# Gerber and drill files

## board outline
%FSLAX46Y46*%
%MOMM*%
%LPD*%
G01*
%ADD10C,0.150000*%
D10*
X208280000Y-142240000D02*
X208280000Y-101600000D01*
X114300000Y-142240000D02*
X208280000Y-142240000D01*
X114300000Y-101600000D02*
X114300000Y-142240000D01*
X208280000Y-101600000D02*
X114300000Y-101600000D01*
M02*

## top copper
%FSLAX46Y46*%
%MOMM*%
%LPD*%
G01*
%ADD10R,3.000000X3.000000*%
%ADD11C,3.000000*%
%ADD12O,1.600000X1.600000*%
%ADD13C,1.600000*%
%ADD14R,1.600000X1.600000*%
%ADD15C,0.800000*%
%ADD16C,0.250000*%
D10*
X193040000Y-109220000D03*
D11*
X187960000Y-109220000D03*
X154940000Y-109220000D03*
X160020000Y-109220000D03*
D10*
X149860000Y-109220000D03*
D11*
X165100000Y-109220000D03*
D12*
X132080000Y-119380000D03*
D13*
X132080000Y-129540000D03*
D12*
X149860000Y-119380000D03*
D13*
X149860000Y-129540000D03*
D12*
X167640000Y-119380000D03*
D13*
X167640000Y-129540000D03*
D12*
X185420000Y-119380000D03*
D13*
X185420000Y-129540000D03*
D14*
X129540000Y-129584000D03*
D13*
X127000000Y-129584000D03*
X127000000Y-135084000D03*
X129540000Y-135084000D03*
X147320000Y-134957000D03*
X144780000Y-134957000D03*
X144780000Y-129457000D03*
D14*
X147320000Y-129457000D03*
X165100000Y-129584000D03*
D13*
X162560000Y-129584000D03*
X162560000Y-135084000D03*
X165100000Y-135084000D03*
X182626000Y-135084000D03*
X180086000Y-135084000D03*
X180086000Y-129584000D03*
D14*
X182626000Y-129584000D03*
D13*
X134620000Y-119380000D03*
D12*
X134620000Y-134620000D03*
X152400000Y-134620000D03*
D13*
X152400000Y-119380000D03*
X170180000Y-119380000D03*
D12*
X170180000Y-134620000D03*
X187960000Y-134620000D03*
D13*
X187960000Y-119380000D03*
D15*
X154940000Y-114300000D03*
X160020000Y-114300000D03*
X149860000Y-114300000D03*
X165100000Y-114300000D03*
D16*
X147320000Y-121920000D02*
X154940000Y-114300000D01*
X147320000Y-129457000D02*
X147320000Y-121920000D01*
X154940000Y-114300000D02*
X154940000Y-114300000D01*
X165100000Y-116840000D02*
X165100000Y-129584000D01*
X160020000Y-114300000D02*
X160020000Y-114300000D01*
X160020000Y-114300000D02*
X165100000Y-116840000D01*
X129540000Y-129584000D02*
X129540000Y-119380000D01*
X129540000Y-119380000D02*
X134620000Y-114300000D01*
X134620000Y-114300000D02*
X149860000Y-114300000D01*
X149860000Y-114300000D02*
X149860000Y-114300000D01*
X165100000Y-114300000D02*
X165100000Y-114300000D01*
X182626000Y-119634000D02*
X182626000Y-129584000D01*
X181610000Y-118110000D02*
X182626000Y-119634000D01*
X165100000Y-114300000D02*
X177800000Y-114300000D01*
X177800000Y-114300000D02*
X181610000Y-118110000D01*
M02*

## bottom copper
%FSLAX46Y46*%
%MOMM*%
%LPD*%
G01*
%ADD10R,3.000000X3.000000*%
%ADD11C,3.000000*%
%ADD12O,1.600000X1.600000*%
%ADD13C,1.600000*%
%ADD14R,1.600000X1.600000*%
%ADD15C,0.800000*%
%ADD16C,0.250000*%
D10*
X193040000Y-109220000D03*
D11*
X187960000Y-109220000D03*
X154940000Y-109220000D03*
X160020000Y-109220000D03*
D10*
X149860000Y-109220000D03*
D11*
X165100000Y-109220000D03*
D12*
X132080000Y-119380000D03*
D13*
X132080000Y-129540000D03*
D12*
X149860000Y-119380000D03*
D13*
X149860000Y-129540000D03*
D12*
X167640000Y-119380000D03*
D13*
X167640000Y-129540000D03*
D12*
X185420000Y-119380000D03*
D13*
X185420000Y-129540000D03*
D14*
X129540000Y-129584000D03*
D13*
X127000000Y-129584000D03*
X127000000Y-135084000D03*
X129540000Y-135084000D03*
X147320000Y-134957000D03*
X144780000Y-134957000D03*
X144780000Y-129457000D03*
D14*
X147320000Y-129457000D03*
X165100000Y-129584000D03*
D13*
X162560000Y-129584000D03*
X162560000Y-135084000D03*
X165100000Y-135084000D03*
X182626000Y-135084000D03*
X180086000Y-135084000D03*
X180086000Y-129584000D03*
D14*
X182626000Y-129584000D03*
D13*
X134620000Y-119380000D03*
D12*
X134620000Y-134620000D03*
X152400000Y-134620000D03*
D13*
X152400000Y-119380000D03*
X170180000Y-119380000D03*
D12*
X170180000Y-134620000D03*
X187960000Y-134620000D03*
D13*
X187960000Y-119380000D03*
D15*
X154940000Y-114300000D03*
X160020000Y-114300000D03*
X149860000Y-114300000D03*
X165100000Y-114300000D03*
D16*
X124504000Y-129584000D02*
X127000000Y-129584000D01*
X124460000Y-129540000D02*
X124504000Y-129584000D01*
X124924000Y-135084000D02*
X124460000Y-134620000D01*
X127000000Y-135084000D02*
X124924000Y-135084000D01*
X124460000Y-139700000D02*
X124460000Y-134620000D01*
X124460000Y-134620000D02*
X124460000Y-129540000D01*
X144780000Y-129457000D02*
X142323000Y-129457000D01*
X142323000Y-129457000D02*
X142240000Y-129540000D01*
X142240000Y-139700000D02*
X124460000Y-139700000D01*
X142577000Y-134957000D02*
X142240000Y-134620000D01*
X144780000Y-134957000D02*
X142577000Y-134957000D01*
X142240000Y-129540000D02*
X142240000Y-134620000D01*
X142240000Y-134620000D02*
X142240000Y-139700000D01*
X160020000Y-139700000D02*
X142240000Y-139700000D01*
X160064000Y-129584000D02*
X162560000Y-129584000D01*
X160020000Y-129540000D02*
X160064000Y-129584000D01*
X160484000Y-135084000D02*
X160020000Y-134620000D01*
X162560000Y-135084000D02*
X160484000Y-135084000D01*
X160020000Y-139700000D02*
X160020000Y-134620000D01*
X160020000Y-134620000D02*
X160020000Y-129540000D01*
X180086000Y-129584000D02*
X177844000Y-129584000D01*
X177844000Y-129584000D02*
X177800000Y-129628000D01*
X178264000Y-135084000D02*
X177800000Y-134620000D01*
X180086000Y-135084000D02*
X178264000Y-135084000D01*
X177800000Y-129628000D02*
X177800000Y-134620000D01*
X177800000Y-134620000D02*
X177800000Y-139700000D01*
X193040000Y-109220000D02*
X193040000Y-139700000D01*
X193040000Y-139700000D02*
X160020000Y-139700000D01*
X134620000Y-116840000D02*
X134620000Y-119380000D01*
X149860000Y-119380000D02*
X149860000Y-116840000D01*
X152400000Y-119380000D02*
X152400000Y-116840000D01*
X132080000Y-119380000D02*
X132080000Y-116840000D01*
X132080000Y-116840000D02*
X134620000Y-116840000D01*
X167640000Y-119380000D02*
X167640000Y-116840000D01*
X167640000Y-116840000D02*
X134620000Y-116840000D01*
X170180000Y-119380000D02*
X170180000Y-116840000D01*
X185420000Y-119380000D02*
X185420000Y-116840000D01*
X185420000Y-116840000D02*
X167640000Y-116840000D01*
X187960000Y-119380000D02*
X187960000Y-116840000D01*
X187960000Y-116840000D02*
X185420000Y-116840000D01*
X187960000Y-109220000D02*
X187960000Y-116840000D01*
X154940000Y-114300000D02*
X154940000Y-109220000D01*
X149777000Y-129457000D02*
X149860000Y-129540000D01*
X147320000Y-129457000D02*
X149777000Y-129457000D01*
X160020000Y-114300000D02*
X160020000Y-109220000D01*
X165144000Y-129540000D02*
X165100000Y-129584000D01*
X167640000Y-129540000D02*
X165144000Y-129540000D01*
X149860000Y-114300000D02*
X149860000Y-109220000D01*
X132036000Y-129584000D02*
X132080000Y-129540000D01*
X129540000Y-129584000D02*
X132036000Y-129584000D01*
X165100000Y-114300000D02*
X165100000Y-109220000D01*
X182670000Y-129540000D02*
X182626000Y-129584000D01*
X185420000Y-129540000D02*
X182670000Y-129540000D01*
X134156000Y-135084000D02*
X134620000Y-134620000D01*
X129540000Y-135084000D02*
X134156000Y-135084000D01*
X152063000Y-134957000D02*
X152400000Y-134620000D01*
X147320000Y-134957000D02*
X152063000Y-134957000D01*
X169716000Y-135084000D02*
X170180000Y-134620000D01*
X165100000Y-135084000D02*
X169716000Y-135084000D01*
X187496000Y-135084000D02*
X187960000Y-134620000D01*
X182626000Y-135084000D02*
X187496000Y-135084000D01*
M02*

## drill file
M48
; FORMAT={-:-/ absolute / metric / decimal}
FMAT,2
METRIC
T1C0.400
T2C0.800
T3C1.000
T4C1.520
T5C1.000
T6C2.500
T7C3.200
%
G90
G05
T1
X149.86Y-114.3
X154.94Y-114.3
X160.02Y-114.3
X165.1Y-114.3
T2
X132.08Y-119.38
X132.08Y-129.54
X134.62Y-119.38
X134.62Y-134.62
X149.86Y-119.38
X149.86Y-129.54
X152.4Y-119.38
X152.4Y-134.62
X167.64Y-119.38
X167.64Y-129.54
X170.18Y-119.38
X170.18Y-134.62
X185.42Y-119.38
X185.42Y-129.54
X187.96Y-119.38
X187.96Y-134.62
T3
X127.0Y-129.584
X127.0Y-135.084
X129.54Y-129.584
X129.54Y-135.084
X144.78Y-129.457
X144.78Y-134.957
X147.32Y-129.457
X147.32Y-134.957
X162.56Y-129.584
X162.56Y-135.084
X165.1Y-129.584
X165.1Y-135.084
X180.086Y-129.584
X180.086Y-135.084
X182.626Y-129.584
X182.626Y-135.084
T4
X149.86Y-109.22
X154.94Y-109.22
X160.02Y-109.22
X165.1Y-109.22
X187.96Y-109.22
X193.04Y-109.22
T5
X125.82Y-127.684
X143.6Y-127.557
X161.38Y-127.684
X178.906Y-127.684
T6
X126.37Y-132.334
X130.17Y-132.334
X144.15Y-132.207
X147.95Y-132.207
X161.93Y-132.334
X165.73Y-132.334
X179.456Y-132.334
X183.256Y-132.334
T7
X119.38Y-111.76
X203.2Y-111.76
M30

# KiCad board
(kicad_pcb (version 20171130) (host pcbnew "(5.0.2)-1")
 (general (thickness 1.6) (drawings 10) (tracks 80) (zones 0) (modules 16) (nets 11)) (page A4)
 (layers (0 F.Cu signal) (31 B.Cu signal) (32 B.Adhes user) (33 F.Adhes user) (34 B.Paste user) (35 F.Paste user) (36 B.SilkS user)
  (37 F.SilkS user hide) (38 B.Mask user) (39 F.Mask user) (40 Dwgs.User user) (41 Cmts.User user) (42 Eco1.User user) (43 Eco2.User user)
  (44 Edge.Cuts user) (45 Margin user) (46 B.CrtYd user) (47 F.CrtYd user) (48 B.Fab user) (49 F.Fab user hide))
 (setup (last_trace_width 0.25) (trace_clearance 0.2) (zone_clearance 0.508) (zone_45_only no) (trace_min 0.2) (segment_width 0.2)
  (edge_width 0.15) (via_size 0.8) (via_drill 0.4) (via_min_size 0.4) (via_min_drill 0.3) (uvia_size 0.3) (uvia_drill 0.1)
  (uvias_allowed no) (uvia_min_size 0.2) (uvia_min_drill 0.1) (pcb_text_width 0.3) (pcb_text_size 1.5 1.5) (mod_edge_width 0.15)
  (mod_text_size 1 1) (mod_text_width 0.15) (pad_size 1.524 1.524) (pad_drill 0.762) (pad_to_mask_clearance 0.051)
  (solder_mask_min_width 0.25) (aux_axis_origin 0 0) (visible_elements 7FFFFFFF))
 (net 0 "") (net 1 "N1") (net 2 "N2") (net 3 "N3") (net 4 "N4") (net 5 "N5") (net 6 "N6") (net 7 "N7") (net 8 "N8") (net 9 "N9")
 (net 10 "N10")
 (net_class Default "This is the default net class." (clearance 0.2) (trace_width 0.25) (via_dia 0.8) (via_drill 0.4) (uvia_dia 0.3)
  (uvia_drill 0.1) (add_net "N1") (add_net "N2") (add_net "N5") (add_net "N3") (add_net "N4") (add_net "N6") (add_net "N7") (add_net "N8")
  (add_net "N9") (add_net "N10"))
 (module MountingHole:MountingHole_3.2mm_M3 (layer F.Cu) (at 203.2 111.76)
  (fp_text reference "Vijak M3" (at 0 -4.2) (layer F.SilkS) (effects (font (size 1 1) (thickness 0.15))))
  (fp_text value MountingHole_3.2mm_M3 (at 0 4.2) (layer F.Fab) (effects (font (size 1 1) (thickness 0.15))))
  (pad 1 np_thru_hole circle (at 0 0) (size 3.2 3.2) (drill 3.2) (layers *.Cu *.Mask)))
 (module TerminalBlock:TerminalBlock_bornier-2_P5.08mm (layer F.Cu) (at 193.04 109.22 180)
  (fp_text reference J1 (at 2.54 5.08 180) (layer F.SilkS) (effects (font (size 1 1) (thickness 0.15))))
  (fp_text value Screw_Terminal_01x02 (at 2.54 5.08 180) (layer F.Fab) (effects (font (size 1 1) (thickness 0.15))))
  (pad 1 thru_hole rect (at 0 0 180) (size 3 3) (drill 1.52) (layers *.Cu *.Mask) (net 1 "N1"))
  (pad 2 thru_hole circle (at 5.08 0 180) (size 3 3) (drill 1.52) (layers *.Cu *.Mask) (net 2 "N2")))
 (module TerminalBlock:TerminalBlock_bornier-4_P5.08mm (layer F.Cu) (at 149.86 109.22)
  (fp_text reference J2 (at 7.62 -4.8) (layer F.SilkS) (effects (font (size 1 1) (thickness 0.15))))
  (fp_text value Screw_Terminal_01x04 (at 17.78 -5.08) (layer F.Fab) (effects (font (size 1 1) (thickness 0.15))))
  (pad 2 thru_hole circle (at 5.08 0) (size 3 3) (drill 1.52) (layers *.Cu *.Mask) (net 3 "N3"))
  (pad 3 thru_hole circle (at 10.16 0) (size 3 3) (drill 1.52) (layers *.Cu *.Mask) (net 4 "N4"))
  (pad 1 thru_hole rect (at 0 0) (size 3 3) (drill 1.52) (layers *.Cu *.Mask) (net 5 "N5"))
  (pad 4 thru_hole circle (at 15.24 0) (size 3 3) (drill 1.52) (layers *.Cu *.Mask) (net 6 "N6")))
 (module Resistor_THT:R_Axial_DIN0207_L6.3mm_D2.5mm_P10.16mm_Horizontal (layer F.Cu) (at 132.08 129.54 90)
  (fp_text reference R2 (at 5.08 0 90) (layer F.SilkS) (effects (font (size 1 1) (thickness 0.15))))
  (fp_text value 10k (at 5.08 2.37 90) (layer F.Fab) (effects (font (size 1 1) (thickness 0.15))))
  (pad 2 thru_hole oval (at 10.16 0 90) (size 1.6 1.6) (drill 0.8) (layers *.Cu *.Mask) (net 2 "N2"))
  (pad 1 thru_hole circle (at 0 0 90) (size 1.6 1.6) (drill 0.8) (layers *.Cu *.Mask) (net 5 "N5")))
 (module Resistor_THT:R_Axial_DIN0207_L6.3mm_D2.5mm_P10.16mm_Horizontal (layer F.Cu) (at 149.86 129.54 90)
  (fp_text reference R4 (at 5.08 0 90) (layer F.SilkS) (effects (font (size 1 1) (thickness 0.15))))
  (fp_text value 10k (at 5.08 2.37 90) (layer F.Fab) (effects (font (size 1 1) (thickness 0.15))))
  (pad 2 thru_hole oval (at 10.16 0 90) (size 1.6 1.6) (drill 0.8) (layers *.Cu *.Mask) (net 2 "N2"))
  (pad 1 thru_hole circle (at 0 0 90) (size 1.6 1.6) (drill 0.8) (layers *.Cu *.Mask) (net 3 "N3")))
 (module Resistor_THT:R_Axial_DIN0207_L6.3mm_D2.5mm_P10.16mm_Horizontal (layer F.Cu) (at 167.64 129.54 90)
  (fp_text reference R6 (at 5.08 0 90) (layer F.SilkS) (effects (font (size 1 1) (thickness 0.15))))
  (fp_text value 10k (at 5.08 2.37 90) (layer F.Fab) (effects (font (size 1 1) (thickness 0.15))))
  (pad 2 thru_hole oval (at 10.16 0 90) (size 1.6 1.6) (drill 0.8) (layers *.Cu *.Mask) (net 2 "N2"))
  (pad 1 thru_hole circle (at 0 0 90) (size 1.6 1.6) (drill 0.8) (layers *.Cu *.Mask) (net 4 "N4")))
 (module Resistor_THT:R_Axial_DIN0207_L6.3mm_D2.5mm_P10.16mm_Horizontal (layer F.Cu) (at 185.42 129.54 90)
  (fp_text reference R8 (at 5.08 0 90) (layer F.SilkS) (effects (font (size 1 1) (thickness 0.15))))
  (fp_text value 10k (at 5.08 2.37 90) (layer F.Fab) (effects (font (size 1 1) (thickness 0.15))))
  (pad 2 thru_hole oval (at 10.16 0 90) (size 1.6 1.6) (drill 0.8) (layers *.Cu *.Mask) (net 2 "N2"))
  (pad 1 thru_hole circle (at 0 0 90) (size 1.6 1.6) (drill 0.8) (layers *.Cu *.Mask) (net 6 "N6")))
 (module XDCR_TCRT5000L (layer F.Cu) (at 128.27 132.334 270)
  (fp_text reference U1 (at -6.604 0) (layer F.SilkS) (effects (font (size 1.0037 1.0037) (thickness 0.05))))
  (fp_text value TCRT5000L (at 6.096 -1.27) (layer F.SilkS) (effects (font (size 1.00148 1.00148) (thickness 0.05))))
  (pad 1 thru_hole rect (at -2.75 -1.27 270) (size 1.6 1.6) (drill 1) (layers *.Cu *.Mask) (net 5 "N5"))
  (pad 2 thru_hole circle (at -2.75 1.27 270) (size 1.6 1.6) (drill 1) (layers *.Cu *.Mask) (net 1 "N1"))
  (pad 3 thru_hole circle (at 2.75 1.27 270) (size 1.6 1.6) (drill 1) (layers *.Cu *.Mask) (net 1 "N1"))
  (pad 4 thru_hole circle (at 2.75 -1.27 270) (size 1.6 1.6) (drill 1) (layers *.Cu *.Mask) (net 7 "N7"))
  (pad Hole np_thru_hole circle (at 0 -1.9 270) (size 2.5 2.5) (drill 2.5) (layers *.Cu *.Mask F.SilkS))
  (pad Hole np_thru_hole circle (at 0 1.9 270) (size 2.5 2.5) (drill 2.5) (layers *.Cu *.Mask F.SilkS))
  (pad Hole np_thru_hole circle (at -4.65 2.45 270) (size 1 1) (drill 1) (layers *.Cu *.Mask F.SilkS)))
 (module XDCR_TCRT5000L (layer F.Cu) (at 146.05 132.207 270)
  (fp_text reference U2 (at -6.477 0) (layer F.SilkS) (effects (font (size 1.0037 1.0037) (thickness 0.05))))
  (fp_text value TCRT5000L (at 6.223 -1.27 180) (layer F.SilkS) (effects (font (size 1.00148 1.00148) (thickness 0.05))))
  (pad Hole np_thru_hole circle (at -4.65 2.45 270) (size 1 1) (drill 1) (layers *.Cu *.Mask F.SilkS))
  (pad Hole np_thru_hole circle (at 0 1.9 270) (size 2.5 2.5) (drill 2.5) (layers *.Cu *.Mask F.SilkS))
  (pad Hole np_thru_hole circle (at 0 -1.9 270) (size 2.5 2.5) (drill 2.5) (layers *.Cu *.Mask F.SilkS))
  (pad 4 thru_hole circle (at 2.75 -1.27 270) (size 1.6 1.6) (drill 1) (layers *.Cu *.Mask) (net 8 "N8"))
  (pad 3 thru_hole circle (at 2.75 1.27 270) (size 1.6 1.6) (drill 1) (layers *.Cu *.Mask) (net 1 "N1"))
  (pad 2 thru_hole circle (at -2.75 1.27 270) (size 1.6 1.6) (drill 1) (layers *.Cu *.Mask) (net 1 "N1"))
  (pad 1 thru_hole rect (at -2.75 -1.27 270) (size 1.6 1.6) (drill 1) (layers *.Cu *.Mask) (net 3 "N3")))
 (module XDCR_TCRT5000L (layer F.Cu) (at 163.83 132.334 270)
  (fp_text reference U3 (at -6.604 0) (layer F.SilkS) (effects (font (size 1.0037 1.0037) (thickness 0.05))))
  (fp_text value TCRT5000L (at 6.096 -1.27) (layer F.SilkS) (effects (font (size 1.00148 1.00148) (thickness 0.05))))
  (pad 1 thru_hole rect (at -2.75 -1.27 270) (size 1.6 1.6) (drill 1) (layers *.Cu *.Mask) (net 4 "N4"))
  (pad 2 thru_hole circle (at -2.75 1.27 270) (size 1.6 1.6) (drill 1) (layers *.Cu *.Mask) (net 1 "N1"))
  (pad 3 thru_hole circle (at 2.75 1.27 270) (size 1.6 1.6) (drill 1) (layers *.Cu *.Mask) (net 1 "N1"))
  (pad 4 thru_hole circle (at 2.75 -1.27 270) (size 1.6 1.6) (drill 1) (layers *.Cu *.Mask) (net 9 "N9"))
  (pad Hole np_thru_hole circle (at 0 -1.9 270) (size 2.5 2.5) (drill 2.5) (layers *.Cu *.Mask F.SilkS))
  (pad Hole np_thru_hole circle (at 0 1.9 270) (size 2.5 2.5) (drill 2.5) (layers *.Cu *.Mask F.SilkS))
  (pad Hole np_thru_hole circle (at -4.65 2.45 270) (size 1 1) (drill 1) (layers *.Cu *.Mask F.SilkS)))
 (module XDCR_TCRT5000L (layer F.Cu) (at 181.356 132.334 270)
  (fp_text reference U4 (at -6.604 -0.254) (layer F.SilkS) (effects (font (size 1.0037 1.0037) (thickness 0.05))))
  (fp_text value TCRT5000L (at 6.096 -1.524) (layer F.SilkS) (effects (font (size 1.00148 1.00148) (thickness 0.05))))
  (pad Hole np_thru_hole circle (at -4.65 2.45 270) (size 1 1) (drill 1) (layers *.Cu *.Mask F.SilkS))
  (pad Hole np_thru_hole circle (at 0 1.9 270) (size 2.5 2.5) (drill 2.5) (layers *.Cu *.Mask F.SilkS))
  (pad Hole np_thru_hole circle (at 0 -1.9 270) (size 2.5 2.5) (drill 2.5) (layers *.Cu *.Mask F.SilkS))
  (pad 4 thru_hole circle (at 2.75 -1.27 270) (size 1.6 1.6) (drill 1) (layers *.Cu *.Mask) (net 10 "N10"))
  (pad 3 thru_hole circle (at 2.75 1.27 270) (size 1.6 1.6) (drill 1) (layers *.Cu *.Mask) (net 1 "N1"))
  (pad 2 thru_hole circle (at -2.75 1.27 270) (size 1.6 1.6) (drill 1) (layers *.Cu *.Mask) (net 1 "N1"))
  (pad 1 thru_hole rect (at -2.75 -1.27 270) (size 1.6 1.6) (drill 1) (layers *.Cu *.Mask) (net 6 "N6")))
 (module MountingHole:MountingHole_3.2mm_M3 (layer F.Cu) (at 119.38 111.76)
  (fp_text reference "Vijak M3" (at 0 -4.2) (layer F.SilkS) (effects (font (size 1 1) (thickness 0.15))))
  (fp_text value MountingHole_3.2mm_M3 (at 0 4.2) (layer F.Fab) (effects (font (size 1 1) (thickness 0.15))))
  (pad 1 np_thru_hole circle (at 0 0) (size 3.2 3.2) (drill 3.2) (layers *.Cu *.Mask)))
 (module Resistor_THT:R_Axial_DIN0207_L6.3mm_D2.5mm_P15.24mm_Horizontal (layer F.Cu) (at 134.62 119.38 270)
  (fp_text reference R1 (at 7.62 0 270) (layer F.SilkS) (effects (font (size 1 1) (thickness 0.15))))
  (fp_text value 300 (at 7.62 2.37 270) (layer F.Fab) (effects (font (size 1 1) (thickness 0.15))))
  (pad 1 thru_hole circle (at 0 0 270) (size 1.6 1.6) (drill 0.8) (layers *.Cu *.Mask) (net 2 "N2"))
  (pad 2 thru_hole oval (at 15.24 0 270) (size 1.6 1.6) (drill 0.8) (layers *.Cu *.Mask) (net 7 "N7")))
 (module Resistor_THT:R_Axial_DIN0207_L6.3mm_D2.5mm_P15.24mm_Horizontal (layer F.Cu) (at 152.4 119.38 270)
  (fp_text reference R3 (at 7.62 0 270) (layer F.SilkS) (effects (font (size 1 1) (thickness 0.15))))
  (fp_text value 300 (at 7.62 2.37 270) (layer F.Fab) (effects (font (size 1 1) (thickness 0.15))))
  (pad 2 thru_hole oval (at 15.24 0 270) (size 1.6 1.6) (drill 0.8) (layers *.Cu *.Mask) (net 8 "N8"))
  (pad 1 thru_hole circle (at 0 0 270) (size 1.6 1.6) (drill 0.8) (layers *.Cu *.Mask) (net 2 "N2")))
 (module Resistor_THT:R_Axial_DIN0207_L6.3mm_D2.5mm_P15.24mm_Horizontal (layer F.Cu) (at 170.18 119.38 270)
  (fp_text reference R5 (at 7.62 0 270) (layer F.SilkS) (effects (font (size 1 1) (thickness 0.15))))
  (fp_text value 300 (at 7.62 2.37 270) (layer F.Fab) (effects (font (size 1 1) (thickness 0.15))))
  (pad 1 thru_hole circle (at 0 0 270) (size 1.6 1.6) (drill 0.8) (layers *.Cu *.Mask) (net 2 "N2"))
  (pad 2 thru_hole oval (at 15.24 0 270) (size 1.6 1.6) (drill 0.8) (layers *.Cu *.Mask) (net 9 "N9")))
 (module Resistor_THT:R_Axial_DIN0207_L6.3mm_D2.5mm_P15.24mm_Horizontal (layer F.Cu) (at 187.96 119.38 270)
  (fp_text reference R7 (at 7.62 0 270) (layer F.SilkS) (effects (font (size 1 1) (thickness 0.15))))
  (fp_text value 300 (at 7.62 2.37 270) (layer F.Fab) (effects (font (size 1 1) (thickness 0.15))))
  (pad 2 thru_hole oval (at 15.24 0 270) (size 1.6 1.6) (drill 0.8) (layers *.Cu *.Mask) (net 10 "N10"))
  (pad 1 thru_hole circle (at 0 0 270) (size 1.6 1.6) (drill 0.8) (layers *.Cu *.Mask) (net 2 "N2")))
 (gr_line (start 208.28 142.24) (end 208.28 101.6) (layer Edge.Cuts) (width 0.15))
 (gr_line (start 114.3 142.24) (end 208.28 142.24) (layer Edge.Cuts) (width 0.15))
 (gr_line (start 114.3 101.6) (end 114.3 142.24) (layer Edge.Cuts) (width 0.15))
 (gr_line (start 208.28 101.6) (end 114.3 101.6) (layer Edge.Cuts) (width 0.15))
 (segment (start 124.504 129.584) (end 127 129.584) (width 0.25) (layer B.Cu) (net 1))
 (segment (start 124.46 129.54) (end 124.504 129.584) (width 0.25) (layer B.Cu) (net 1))
 (segment (start 124.924 135.084) (end 124.46 134.62) (width 0.25) (layer B.Cu) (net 1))
 (segment (start 127 135.084) (end 124.924 135.084) (width 0.25) (layer B.Cu) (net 1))
 (segment (start 124.46 139.7) (end 124.46 134.62) (width 0.25) (layer B.Cu) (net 1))
 (segment (start 124.46 134.62) (end 124.46 129.54) (width 0.25) (layer B.Cu) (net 1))
 (segment (start 144.78 129.457) (end 142.323 129.457) (width 0.25) (layer B.Cu) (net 1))
 (segment (start 142.323 129.457) (end 142.24 129.54) (width 0.25) (layer B.Cu) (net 1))
 (segment (start 142.24 139.7) (end 124.46 139.7) (width 0.25) (layer B.Cu) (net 1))
 (segment (start 142.577 134.957) (end 142.24 134.62) (width 0.25) (layer B.Cu) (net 1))
 (segment (start 144.78 134.957) (end 142.577 134.957) (width 0.25) (layer B.Cu) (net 1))
 (segment (start 142.24 129.54) (end 142.24 134.62) (width 0.25) (layer B.Cu) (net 1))
 (segment (start 142.24 134.62) (end 142.24 139.7) (width 0.25) (layer B.Cu) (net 1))
 (segment (start 160.02 139.7) (end 142.24 139.7) (width 0.25) (layer B.Cu) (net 1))
 (segment (start 160.064 129.584) (end 162.56 129.584) (width 0.25) (layer B.Cu) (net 1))
 (segment (start 160.02 129.54) (end 160.064 129.584) (width 0.25) (layer B.Cu) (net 1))
 (segment (start 160.484 135.084) (end 160.02 134.62) (width 0.25) (layer B.Cu) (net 1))
 (segment (start 162.56 135.084) (end 160.484 135.084) (width 0.25) (layer B.Cu) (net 1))
 (segment (start 160.02 139.7) (end 160.02 134.62) (width 0.25) (layer B.Cu) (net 1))
 (segment (start 160.02 134.62) (end 160.02 129.54) (width 0.25) (layer B.Cu) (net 1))
 (segment (start 180.086 129.584) (end 177.844 129.584) (width 0.25) (layer B.Cu) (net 1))
 (segment (start 177.844 129.584) (end 177.8 129.628) (width 0.25) (layer B.Cu) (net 1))
 (segment (start 178.264 135.084) (end 177.8 134.62) (width 0.25) (layer B.Cu) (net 1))
 (segment (start 180.086 135.084) (end 178.264 135.084) (width 0.25) (layer B.Cu) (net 1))
 (segment (start 177.8 129.628) (end 177.8 134.62) (width 0.25) (layer B.Cu) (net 1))
 (segment (start 177.8 134.62) (end 177.8 139.7) (width 0.25) (layer B.Cu) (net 1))
 (segment (start 193.04 109.22) (end 193.04 139.7) (width 0.25) (layer B.Cu) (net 1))
 (segment (start 193.04 139.7) (end 160.02 139.7) (width 0.25) (layer B.Cu) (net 1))
 (segment (start 134.62 116.84) (end 134.62 119.38) (width 0.25) (layer B.Cu) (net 2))
 (segment (start 149.86 119.38) (end 149.86 116.84) (width 0.25) (layer B.Cu) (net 2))
 (segment (start 152.4 119.38) (end 152.4 116.84) (width 0.25) (layer B.Cu) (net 2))
 (segment (start 132.08 119.38) (end 132.08 116.84) (width 0.25) (layer B.Cu) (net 2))
 (segment (start 132.08 116.84) (end 134.62 116.84) (width 0.25) (layer B.Cu) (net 2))
 (segment (start 167.64 119.38) (end 167.64 116.84) (width 0.25) (layer B.Cu) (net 2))
 (segment (start 167.64 116.84) (end 134.62 116.84) (width 0.25) (layer B.Cu) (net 2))
 (segment (start 170.18 119.38) (end 170.18 116.84) (width 0.25) (layer B.Cu) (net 2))
 (segment (start 185.42 119.38) (end 185.42 116.84) (width 0.25) (layer B.Cu) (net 2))
 (segment (start 185.42 116.84) (end 167.64 116.84) (width 0.25) (layer B.Cu) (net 2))
 (segment (start 187.96 119.38) (end 187.96 116.84) (width 0.25) (layer B.Cu) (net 2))
 (segment (start 187.96 116.84) (end 185.42 116.84) (width 0.25) (layer B.Cu) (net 2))
 (segment (start 187.96 109.22) (end 187.96 116.84) (width 0.25) (layer B.Cu) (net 2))
 (segment (start 147.32 121.92) (end 154.94 114.3) (width 0.25) (layer F.Cu) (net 3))
 (segment (start 147.32 129.457) (end 147.32 121.92) (width 0.25) (layer F.Cu) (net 3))
 (segment (start 154.94 114.3) (end 154.94 114.3) (width 0.25) (layer F.Cu) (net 3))
 (via (at 154.94 114.3) (size 0.8) (drill 0.4) (layers F.Cu B.Cu) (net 3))
 (segment (start 154.94 114.3) (end 154.94 109.22) (width 0.25) (layer B.Cu) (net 3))
 (segment (start 149.777 129.457) (end 149.86 129.54) (width 0.25) (layer B.Cu) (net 3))
 (segment (start 147.32 129.457) (end 149.777 129.457) (width 0.25) (layer B.Cu) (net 3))
 (segment (start 165.1 116.84) (end 165.1 129.584) (width 0.25) (layer F.Cu) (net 4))
 (segment (start 160.02 114.3) (end 160.02 114.3) (width 0.25) (layer F.Cu) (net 4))
 (segment (start 160.02 114.3) (end 165.1 116.84) (width 0.25) (layer F.Cu) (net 4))
 (via (at 160.02 114.3) (size 0.8) (drill 0.4) (layers F.Cu B.Cu) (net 4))
 (segment (start 160.02 114.3) (end 160.02 109.22) (width 0.25) (layer B.Cu) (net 4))
 (segment (start 165.144 129.54) (end 165.1 129.584) (width 0.25) (layer B.Cu) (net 4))
 (segment (start 167.64 129.54) (end 165.144 129.54) (width 0.25) (layer B.Cu) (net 4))
 (segment (start 129.54 129.584) (end 129.54 119.38) (width 0.25) (layer F.Cu) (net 5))
 (segment (start 129.54 119.38) (end 134.62 114.3) (width 0.25) (layer F.Cu) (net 5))
 (segment (start 134.62 114.3) (end 149.86 114.3) (width 0.25) (layer F.Cu) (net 5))
 (segment (start 149.86 114.3) (end 149.86 114.3) (width 0.25) (layer F.Cu) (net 5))
 (via (at 149.86 114.3) (size 0.8) (drill 0.4) (layers F.Cu B.Cu) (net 5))
 (segment (start 149.86 114.3) (end 149.86 109.22) (width 0.25) (layer B.Cu) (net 5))
 (segment (start 132.036 129.584) (end 132.08 129.54) (width 0.25) (layer B.Cu) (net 5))
 (segment (start 129.54 129.584) (end 132.036 129.584) (width 0.25) (layer B.Cu) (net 5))
 (segment (start 165.1 114.3) (end 165.1 114.3) (width 0.25) (layer F.Cu) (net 6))
 (via (at 165.1 114.3) (size 0.8) (drill 0.4) (layers F.Cu B.Cu) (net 6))
 (segment (start 165.1 114.3) (end 165.1 109.22) (width 0.25) (layer B.Cu) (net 6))
 (segment (start 182.626 119.634) (end 182.626 129.584) (width 0.25) (layer F.Cu) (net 6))
 (segment (start 181.61 118.11) (end 182.626 119.634) (width 0.25) (layer F.Cu) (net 6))
 (segment (start 165.1 114.3) (end 177.8 114.3) (width 0.25) (layer F.Cu) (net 6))
 (segment (start 177.8 114.3) (end 181.61 118.11) (width 0.25) (layer F.Cu) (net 6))
 (segment (start 182.67 129.54) (end 182.626 129.584) (width 0.25) (layer B.Cu) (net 6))
 (segment (start 185.42 129.54) (end 182.67 129.54) (width 0.25) (layer B.Cu) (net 6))
 (segment (start 134.156 135.084) (end 134.62 134.62) (width 0.25) (layer B.Cu) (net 7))
 (segment (start 129.54 135.084) (end 134.156 135.084) (width 0.25) (layer B.Cu) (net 7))
 (segment (start 152.063 134.957) (end 152.4 134.62) (width 0.25) (layer B.Cu) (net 8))
 (segment (start 147.32 134.957) (end 152.063 134.957) (width 0.25) (layer B.Cu) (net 8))
 (segment (start 169.716 135.084) (end 170.18 134.62) (width 0.25) (layer B.Cu) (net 9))
 (segment (start 165.1 135.084) (end 169.716 135.084) (width 0.25) (layer B.Cu) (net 9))
 (segment (start 187.496 135.084) (end 187.96 134.62) (width 0.25) (layer B.Cu) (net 10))
 (segment (start 182.626 135.084) (end 187.496 135.084) (width 0.25) (layer B.Cu) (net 10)))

